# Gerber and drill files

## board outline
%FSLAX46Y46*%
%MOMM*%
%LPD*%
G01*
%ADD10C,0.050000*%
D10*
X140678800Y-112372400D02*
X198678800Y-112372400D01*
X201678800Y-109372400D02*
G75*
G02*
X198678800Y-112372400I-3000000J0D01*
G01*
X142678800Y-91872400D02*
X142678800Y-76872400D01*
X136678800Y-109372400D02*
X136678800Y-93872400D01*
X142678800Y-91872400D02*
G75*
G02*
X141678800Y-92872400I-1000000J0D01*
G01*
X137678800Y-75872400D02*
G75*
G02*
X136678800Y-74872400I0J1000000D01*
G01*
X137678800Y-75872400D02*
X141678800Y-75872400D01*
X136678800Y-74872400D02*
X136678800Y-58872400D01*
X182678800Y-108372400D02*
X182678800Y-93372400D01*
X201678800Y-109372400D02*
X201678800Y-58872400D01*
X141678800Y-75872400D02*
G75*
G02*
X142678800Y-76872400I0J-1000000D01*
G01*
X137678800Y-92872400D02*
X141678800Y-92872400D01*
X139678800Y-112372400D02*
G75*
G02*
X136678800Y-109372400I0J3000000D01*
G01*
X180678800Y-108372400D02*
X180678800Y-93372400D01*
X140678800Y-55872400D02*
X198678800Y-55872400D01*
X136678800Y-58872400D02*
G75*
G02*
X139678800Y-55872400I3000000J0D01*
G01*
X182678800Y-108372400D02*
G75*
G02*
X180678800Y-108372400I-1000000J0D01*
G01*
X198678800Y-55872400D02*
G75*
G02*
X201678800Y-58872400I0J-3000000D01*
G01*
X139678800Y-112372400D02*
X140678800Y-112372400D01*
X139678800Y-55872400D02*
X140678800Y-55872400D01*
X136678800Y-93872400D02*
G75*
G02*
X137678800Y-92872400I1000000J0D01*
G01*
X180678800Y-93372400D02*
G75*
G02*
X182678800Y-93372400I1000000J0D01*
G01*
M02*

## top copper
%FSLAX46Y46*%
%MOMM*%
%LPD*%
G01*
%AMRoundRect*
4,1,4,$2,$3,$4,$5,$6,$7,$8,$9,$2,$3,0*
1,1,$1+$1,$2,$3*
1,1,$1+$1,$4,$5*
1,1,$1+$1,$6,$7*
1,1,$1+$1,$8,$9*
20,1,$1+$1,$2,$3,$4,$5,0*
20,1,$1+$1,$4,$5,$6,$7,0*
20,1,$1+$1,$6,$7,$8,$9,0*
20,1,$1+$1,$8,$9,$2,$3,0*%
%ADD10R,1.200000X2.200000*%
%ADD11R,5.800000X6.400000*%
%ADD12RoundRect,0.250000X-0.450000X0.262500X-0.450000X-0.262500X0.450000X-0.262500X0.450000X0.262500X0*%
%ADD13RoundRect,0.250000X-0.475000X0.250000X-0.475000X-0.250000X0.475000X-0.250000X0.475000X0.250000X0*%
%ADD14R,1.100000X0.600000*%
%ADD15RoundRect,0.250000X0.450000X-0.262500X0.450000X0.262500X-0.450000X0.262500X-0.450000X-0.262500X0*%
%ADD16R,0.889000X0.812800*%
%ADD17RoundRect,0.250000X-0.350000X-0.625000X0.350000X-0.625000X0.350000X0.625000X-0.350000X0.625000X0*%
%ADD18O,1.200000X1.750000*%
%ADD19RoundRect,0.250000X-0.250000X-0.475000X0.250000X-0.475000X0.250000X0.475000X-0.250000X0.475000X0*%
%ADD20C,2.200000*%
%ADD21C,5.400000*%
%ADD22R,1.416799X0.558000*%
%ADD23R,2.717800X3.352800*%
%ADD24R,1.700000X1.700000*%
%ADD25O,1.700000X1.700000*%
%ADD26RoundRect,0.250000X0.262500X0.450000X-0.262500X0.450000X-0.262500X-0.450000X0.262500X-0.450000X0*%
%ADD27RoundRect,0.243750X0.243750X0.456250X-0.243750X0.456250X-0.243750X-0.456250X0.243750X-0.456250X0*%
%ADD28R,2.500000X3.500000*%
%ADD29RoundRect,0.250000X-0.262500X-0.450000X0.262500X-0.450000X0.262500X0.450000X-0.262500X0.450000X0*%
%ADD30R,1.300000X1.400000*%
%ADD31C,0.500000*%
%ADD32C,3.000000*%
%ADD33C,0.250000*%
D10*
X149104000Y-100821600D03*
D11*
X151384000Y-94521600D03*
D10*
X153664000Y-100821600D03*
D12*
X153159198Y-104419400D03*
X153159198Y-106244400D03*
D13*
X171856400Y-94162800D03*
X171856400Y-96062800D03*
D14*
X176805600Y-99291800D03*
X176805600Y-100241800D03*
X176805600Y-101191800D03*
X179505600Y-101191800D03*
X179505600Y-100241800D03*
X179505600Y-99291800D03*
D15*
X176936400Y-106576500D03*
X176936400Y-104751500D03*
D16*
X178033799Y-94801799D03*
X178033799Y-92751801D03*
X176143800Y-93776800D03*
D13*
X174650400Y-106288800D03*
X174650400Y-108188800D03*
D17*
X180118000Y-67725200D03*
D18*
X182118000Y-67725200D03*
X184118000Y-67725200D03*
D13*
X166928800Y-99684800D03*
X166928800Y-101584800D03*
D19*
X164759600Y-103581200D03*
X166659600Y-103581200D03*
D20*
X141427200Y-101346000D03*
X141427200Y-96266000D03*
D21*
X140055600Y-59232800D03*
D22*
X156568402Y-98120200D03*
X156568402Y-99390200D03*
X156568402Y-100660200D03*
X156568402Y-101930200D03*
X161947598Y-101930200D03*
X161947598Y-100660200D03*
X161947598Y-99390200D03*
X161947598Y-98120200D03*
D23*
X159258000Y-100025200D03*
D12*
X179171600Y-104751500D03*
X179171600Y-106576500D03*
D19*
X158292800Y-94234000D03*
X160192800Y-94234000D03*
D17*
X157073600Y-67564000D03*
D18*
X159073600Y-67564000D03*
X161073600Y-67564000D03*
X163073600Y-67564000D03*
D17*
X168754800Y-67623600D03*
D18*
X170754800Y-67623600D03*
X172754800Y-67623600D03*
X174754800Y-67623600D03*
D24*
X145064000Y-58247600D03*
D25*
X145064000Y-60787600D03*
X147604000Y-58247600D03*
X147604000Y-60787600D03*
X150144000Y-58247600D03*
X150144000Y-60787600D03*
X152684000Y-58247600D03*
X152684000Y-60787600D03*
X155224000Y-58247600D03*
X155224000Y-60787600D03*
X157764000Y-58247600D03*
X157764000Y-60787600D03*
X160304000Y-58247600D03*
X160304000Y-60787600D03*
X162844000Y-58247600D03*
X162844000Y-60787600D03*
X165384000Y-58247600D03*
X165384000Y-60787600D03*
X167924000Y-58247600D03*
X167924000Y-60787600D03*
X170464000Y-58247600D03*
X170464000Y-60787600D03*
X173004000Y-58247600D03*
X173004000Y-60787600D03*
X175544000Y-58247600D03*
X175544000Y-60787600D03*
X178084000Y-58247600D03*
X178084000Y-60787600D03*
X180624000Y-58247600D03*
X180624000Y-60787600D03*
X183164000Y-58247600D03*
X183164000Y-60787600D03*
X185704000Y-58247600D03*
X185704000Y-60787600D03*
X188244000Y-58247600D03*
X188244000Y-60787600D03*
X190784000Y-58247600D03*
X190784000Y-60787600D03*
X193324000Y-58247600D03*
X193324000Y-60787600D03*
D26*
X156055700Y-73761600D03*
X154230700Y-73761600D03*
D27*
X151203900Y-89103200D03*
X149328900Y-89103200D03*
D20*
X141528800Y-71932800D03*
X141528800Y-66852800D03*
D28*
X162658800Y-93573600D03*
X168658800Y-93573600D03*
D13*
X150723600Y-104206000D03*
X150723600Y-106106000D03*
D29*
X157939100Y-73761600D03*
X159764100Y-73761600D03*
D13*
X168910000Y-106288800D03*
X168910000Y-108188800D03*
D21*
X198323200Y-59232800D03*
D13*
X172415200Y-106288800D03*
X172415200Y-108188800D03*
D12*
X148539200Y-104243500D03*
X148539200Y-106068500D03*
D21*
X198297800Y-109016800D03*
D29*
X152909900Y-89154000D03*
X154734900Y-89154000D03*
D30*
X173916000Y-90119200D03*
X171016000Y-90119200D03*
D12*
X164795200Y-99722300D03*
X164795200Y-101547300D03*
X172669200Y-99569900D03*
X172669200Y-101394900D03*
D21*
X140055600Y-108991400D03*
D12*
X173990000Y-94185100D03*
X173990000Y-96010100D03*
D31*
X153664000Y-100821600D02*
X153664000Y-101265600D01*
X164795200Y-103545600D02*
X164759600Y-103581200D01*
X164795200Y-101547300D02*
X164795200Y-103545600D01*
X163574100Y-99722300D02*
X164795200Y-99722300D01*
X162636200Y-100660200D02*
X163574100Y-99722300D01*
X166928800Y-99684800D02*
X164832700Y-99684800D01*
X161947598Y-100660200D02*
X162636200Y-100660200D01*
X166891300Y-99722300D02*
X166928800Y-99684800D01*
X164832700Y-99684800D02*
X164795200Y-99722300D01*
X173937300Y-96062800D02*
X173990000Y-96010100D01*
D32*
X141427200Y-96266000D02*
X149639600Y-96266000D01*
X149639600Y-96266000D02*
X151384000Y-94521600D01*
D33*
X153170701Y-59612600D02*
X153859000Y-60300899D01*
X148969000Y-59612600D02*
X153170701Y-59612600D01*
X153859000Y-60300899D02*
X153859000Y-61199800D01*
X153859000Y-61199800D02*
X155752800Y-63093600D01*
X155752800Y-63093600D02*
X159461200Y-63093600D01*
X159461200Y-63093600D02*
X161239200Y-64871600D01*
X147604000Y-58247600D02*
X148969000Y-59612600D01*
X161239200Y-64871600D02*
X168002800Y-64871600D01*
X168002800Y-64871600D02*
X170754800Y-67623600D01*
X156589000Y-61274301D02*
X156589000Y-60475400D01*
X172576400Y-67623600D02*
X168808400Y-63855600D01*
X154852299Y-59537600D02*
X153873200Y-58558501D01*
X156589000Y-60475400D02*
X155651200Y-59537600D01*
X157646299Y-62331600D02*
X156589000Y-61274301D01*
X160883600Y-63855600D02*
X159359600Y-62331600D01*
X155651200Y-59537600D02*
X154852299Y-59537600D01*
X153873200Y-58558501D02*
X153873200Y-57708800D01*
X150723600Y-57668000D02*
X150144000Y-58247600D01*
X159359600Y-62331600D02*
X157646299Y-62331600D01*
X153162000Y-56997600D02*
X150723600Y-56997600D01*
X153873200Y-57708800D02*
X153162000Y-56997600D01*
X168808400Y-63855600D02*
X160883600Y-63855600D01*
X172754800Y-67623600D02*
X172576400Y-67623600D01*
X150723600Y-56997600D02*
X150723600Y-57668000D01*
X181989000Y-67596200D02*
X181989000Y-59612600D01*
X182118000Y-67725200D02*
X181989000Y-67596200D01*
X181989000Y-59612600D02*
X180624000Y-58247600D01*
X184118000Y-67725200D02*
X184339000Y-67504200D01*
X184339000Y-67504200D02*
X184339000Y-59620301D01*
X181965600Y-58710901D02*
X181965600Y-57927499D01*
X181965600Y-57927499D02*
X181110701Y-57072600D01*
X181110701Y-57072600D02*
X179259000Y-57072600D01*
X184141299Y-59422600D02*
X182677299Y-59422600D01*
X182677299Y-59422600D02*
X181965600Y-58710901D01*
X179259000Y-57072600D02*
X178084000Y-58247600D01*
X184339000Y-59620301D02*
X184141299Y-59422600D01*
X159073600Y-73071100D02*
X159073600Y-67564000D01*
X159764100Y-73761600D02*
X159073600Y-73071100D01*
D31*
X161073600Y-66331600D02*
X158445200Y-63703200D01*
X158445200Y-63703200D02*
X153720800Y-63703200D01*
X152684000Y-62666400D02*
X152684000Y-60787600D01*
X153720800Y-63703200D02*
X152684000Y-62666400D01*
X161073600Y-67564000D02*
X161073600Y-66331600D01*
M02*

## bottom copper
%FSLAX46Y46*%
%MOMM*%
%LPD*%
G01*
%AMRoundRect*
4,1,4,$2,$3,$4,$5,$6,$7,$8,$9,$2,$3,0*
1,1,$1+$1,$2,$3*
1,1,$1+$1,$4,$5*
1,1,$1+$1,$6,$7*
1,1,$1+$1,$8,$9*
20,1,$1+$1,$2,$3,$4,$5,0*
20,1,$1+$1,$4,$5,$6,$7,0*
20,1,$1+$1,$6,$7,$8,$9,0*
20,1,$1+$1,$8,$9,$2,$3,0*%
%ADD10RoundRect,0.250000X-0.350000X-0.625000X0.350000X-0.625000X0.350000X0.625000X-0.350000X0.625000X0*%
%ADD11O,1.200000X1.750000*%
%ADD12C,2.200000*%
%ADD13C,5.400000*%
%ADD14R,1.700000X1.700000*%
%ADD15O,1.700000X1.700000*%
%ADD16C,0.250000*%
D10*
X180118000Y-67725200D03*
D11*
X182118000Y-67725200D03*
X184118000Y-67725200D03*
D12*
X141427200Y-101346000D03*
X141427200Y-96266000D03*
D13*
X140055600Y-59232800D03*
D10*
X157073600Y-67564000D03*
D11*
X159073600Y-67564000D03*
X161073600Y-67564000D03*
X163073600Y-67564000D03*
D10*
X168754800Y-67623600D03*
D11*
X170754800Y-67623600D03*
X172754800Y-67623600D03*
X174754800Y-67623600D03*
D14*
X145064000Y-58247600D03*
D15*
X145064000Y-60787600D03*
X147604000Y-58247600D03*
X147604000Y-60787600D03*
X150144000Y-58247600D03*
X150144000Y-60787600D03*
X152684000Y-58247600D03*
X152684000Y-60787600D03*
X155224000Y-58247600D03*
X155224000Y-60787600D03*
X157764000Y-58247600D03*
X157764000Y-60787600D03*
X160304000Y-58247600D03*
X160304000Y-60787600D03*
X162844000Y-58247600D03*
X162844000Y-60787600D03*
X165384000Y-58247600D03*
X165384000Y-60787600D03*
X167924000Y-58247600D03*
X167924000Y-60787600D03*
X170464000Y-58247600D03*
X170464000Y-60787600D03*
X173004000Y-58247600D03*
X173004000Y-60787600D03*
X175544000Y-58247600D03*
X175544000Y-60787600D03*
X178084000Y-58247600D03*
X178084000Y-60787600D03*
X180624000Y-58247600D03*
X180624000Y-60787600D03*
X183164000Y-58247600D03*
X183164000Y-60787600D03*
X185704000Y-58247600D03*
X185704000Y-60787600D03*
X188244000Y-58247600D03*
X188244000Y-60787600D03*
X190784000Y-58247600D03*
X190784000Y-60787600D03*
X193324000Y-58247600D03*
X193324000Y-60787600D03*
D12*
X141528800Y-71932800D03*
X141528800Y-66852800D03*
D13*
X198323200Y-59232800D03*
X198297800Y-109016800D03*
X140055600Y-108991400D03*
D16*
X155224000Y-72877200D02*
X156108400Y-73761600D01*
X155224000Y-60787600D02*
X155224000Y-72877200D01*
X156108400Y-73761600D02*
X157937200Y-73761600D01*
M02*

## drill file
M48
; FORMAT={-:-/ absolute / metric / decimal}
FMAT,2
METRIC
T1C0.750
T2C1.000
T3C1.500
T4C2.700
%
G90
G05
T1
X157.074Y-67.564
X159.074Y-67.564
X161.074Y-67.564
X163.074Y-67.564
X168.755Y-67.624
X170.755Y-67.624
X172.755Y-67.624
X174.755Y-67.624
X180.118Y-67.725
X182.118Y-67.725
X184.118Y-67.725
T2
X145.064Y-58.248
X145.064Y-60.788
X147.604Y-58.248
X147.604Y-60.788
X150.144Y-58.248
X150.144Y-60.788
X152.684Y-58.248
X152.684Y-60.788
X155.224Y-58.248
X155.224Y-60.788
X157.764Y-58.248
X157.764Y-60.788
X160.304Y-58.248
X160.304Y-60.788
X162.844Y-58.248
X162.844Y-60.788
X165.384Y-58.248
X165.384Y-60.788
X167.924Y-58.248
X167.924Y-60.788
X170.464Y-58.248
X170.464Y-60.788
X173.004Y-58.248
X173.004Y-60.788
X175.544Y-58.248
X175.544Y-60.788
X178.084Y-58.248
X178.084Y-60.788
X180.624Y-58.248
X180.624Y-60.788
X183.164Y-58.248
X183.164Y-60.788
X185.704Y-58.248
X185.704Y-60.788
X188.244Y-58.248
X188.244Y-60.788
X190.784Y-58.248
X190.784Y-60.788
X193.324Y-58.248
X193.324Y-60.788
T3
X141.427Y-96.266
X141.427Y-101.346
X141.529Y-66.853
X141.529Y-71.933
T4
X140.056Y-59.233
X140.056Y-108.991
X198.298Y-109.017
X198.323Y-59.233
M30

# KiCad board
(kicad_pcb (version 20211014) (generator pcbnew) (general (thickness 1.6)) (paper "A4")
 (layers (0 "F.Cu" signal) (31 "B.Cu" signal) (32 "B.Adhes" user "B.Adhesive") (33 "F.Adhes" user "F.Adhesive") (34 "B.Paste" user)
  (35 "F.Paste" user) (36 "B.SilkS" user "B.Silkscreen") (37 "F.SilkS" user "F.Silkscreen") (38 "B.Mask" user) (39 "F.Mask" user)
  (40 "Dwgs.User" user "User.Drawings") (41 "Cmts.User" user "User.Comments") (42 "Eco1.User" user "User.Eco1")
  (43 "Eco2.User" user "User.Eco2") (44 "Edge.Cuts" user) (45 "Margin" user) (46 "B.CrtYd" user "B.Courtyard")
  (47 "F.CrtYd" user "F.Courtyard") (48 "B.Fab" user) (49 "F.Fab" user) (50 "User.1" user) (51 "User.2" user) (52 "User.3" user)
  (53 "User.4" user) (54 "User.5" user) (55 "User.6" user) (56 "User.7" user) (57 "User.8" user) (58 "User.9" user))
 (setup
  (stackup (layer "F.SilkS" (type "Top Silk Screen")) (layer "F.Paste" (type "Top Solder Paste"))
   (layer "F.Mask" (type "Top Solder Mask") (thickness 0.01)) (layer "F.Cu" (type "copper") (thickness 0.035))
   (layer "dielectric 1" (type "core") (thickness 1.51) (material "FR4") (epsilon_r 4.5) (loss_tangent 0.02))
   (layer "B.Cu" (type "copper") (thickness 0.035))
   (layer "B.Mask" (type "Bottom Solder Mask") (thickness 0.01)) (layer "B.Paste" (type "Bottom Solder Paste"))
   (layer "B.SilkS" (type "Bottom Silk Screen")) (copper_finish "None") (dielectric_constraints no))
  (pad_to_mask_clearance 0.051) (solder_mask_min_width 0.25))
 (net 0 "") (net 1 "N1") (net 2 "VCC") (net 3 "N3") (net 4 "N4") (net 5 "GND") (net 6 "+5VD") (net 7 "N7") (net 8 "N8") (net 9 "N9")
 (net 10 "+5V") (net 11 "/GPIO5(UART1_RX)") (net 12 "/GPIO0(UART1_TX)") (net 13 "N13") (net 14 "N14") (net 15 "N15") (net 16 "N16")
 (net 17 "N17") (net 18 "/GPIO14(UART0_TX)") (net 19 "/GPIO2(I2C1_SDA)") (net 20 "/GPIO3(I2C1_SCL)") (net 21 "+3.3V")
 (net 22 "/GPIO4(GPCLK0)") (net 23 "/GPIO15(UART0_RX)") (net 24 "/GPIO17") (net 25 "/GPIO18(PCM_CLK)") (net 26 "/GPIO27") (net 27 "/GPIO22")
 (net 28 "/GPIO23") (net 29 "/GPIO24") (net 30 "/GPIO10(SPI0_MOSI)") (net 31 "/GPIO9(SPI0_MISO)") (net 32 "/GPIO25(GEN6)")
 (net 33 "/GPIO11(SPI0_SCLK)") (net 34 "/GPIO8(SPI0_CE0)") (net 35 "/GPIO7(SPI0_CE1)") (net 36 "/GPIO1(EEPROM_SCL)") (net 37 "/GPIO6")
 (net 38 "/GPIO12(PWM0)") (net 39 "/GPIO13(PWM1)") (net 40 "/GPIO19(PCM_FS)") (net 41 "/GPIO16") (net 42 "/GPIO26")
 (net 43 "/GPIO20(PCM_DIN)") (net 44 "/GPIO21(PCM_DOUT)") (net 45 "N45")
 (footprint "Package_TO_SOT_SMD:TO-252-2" (layer "F.Cu") (at 151.384 96.6216 90)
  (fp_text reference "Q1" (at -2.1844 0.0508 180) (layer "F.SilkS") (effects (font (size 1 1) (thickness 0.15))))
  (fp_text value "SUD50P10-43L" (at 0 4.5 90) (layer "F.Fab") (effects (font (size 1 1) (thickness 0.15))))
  (pad "" smd rect (at 0.425 1.525 90) (size 3.05 2.75) (layers "F.Paste"))
  (pad "" smd rect (at 3.775 1.525 90) (size 3.05 2.75) (layers "F.Paste"))
  (pad "" smd rect (at 3.775 -1.525 90) (size 3.05 2.75) (layers "F.Paste"))
  (pad "" smd rect (at 0.425 -1.525 90) (size 3.05 2.75) (layers "F.Paste"))
  (pad "1" smd rect (at -4.2 -2.28 90) (size 2.2 1.2) (layers "F.Cu" "F.Paste" "F.Mask") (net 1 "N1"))
  (pad "2" smd rect (at 2.1 0 90) (size 6.4 5.8) (layers "F.Cu" "F.Mask") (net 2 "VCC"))
  (pad "3" smd rect (at -4.2 2.28 90) (size 2.2 1.2) (layers "F.Cu" "F.Paste" "F.Mask") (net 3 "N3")))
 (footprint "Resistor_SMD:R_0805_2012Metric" (layer "F.Cu") (at 153.159198 105.3319 -90)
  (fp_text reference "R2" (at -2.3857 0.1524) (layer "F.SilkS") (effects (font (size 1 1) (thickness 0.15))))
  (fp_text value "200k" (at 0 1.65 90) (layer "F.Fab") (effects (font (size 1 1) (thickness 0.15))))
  (pad "1" smd roundrect (at -0.9125 0 270) (size 1.025 1.4) (layers "F.Cu" "F.Paste" "F.Mask") (roundrect_rratio 0.243902) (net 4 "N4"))
  (pad "2" smd roundrect (at 0.9125 0 270) (size 1.025 1.4) (layers "F.Cu" "F.Paste" "F.Mask") (roundrect_rratio 0.243902) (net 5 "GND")))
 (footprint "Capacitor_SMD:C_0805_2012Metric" (layer "F.Cu") (at 171.8564 95.1128 -90)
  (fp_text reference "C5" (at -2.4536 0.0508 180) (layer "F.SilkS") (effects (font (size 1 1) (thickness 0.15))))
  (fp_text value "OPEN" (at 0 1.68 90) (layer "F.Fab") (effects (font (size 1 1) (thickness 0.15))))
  (pad "1" smd roundrect (at -0.95 0 270) (size 1 1.45) (layers "F.Cu" "F.Paste" "F.Mask") (roundrect_rratio 0.25) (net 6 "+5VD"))
  (pad "2" smd roundrect (at 0.95 0 270) (size 1 1.45) (layers "F.Cu" "F.Paste" "F.Mask") (roundrect_rratio 0.25) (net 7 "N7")))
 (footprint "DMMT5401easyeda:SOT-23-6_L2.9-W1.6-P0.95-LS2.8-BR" (layer "F.Cu") (at 178.1556 100.2418 180)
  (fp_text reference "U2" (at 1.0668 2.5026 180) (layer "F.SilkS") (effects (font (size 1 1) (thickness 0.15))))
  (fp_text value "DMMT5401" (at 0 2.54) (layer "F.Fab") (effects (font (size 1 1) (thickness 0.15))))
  (pad "1" smd rect (at 1.35 0.95 180) (size 1.1 0.6) (layers "F.Cu" "F.Paste" "F.Mask") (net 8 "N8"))
  (pad "2" smd rect (at 1.35 0 180) (size 1.1 0.6) (layers "F.Cu" "F.Paste" "F.Mask") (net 8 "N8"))
  (pad "3" smd rect (at 1.35 -0.95 180) (size 1.1 0.6) (layers "F.Cu" "F.Paste" "F.Mask") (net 8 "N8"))
  (pad "4" smd rect (at -1.35 -0.95 180) (size 1.1 0.6) (layers "F.Cu" "F.Paste" "F.Mask") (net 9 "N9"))
  (pad "5" smd rect (at -1.35 0 180) (size 1.1 0.6) (layers "F.Cu" "F.Paste" "F.Mask") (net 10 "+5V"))
  (pad "6" smd rect (at -1.35 0.95 180) (size 1.1 0.6) (layers "F.Cu" "F.Paste" "F.Mask") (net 6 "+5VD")))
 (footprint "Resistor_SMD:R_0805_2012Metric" (layer "F.Cu") (at 176.9364 105.664 90)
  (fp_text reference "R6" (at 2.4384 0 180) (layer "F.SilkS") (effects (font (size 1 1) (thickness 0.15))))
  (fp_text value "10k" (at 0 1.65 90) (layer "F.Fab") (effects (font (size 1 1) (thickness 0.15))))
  (pad "1" smd roundrect (at -0.9125 0 90) (size 1.025 1.4) (layers "F.Cu" "F.Paste" "F.Mask") (roundrect_rratio 0.243902) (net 5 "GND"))
  (pad "2" smd roundrect (at 0.9125 0 90) (size 1.025 1.4) (layers "F.Cu" "F.Paste" "F.Mask") (roundrect_rratio 0.243902) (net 8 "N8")))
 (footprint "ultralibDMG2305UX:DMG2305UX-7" (layer "F.Cu") (at 177.0888 93.7768 90)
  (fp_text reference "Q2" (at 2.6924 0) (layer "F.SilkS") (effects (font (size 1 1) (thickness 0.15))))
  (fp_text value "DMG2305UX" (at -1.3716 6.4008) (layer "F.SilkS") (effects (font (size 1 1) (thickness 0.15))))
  (pad "1" smd rect (at -1.024999 0.944999 90) (size 0.8128 0.889) (layers "F.Cu" "F.Paste" "F.Mask") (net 9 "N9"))
  (pad "2" smd rect (at 1.024999 0.944999 90) (size 0.8128 0.889) (layers "F.Cu" "F.Paste" "F.Mask") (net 10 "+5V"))
  (pad "3" smd rect (at 0 -0.945 90) (size 0.8128 0.889) (layers "F.Cu" "F.Paste" "F.Mask") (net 6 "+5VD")))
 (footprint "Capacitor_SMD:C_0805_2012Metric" (layer "F.Cu") (at 174.6504 107.2388 -90)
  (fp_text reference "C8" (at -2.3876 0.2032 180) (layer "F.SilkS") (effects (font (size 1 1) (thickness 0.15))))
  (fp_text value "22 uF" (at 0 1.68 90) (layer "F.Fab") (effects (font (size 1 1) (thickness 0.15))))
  (pad "1" smd roundrect (at -0.95 0 270) (size 1 1.45) (layers "F.Cu" "F.Paste" "F.Mask") (roundrect_rratio 0.25) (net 6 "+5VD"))
  (pad "2" smd roundrect (at 0.95 0 270) (size 1 1.45) (layers "F.Cu" "F.Paste" "F.Mask") (roundrect_rratio 0.25) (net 5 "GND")))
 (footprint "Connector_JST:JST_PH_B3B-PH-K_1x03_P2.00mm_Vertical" (layer "F.Cu") (at 180.118 67.7252)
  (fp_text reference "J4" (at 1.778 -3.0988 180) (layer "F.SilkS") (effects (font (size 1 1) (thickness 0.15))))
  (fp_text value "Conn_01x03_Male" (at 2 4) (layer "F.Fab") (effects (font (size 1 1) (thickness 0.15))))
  (pad "1" thru_hole roundrect (at 0 0) (size 1.2 1.75) (drill 0.75) (layers *.Cu *.Mask) (roundrect_rratio 0.208333) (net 5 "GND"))
  (pad "2" thru_hole oval (at 2 0) (size 1.2 1.75) (drill 0.75) (layers *.Cu *.Mask) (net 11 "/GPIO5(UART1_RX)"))
  (pad "3" thru_hole oval (at 4 0) (size 1.2 1.75) (drill 0.75) (layers *.Cu *.Mask) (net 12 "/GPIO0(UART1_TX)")))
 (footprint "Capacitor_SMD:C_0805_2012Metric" (layer "F.Cu") (at 166.9288 100.6348 -90)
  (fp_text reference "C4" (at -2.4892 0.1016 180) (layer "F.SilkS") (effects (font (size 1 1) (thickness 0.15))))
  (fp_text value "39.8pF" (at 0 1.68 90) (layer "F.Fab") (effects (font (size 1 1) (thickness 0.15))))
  (pad "1" smd roundrect (at -0.95 0 270) (size 1 1.45) (layers "F.Cu" "F.Paste" "F.Mask") (roundrect_rratio 0.25) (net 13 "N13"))
  (pad "2" smd roundrect (at 0.95 0 270) (size 1 1.45) (layers "F.Cu" "F.Paste" "F.Mask") (roundrect_rratio 0.25) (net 5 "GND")))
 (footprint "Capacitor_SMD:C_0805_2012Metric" (layer "F.Cu") (at 165.7096 103.5812)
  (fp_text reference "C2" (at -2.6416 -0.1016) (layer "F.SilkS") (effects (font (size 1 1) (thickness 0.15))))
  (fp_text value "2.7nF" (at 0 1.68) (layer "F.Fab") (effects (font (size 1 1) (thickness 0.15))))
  (pad "1" smd roundrect (at -0.95 0) (size 1 1.45) (layers "F.Cu" "F.Paste" "F.Mask") (roundrect_rratio 0.25) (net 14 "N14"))
  (pad "2" smd roundrect (at 0.95 0) (size 1 1.45) (layers "F.Cu" "F.Paste" "F.Mask") (roundrect_rratio 0.25) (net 5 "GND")))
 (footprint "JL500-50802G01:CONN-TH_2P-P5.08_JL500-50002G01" (layer "F.Cu") (at 141.4272 98.806 90)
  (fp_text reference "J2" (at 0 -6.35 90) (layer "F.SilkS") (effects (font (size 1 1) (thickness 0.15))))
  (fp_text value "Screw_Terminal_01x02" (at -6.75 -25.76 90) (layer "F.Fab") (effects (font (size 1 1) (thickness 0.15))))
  (pad "1" thru_hole circle (at -2.54 0 90) (size 2.2 2.2) (drill 1.500022) (layers *.Cu *.Mask) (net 5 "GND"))
  (pad "2" thru_hole circle (at 2.54 0 90) (size 2.2 2.2) (drill 1.500022) (layers *.Cu *.Mask) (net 2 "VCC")))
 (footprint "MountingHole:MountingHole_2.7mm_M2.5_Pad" (layer "F.Cu") (at 140.0556 59.2328)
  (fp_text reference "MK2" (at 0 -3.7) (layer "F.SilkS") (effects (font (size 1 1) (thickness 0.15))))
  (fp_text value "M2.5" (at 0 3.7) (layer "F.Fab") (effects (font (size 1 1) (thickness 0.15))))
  (pad "1" thru_hole circle (at 0 0) (size 5.4 5.4) (drill 2.7) (layers *.Cu *.Mask)))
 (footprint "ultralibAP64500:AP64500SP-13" (layer "F.Cu") (at 159.258 100.0252)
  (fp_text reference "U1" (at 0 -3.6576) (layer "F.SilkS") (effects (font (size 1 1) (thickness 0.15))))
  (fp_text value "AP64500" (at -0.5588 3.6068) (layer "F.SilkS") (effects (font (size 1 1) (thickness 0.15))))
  (pad "1" smd rect (at -2.689598 -1.905) (size 1.416799 0.558) (layers "F.Cu" "F.Paste" "F.Mask") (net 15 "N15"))
  (pad "2" smd rect (at -2.689598 -0.635) (size 1.416799 0.558) (layers "F.Cu" "F.Paste" "F.Mask") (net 3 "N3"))
  (pad "3" smd rect (at -2.689598 0.635) (size 1.416799 0.558) (layers "F.Cu" "F.Paste" "F.Mask") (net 3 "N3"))
  (pad "4" smd rect (at -2.689598 1.905) (size 1.416799 0.558) (layers "F.Cu" "F.Paste" "F.Mask") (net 4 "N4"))
  (pad "5" smd rect (at 2.689598 1.905) (size 1.416799 0.558) (layers "F.Cu" "F.Paste" "F.Mask") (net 7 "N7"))
  (pad "6" smd rect (at 2.689598 0.635) (size 1.416799 0.558) (layers "F.Cu" "F.Paste" "F.Mask") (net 13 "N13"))
  (pad "7" smd rect (at 2.689598 -0.635) (size 1.416799 0.558) (layers "F.Cu" "F.Paste" "F.Mask") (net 5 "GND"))
  (pad "8" smd rect (at 2.689598 -1.905) (size 1.416799 0.558) (layers "F.Cu" "F.Paste" "F.Mask") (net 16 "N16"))
  (pad "EPAD" smd rect (at 0 0) (size 2.7178 3.3528) (layers "F.Cu" "F.Paste" "F.Mask")))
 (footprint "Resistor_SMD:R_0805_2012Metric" (layer "F.Cu") (at 179.1716 105.664 -90)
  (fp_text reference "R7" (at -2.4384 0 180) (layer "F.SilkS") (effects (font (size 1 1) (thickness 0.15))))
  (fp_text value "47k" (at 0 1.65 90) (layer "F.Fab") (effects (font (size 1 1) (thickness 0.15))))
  (pad "1" smd roundrect (at -0.9125 0 270) (size 1.025 1.4) (layers "F.Cu" "F.Paste" "F.Mask") (roundrect_rratio 0.243902) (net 9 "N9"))
  (pad "2" smd roundrect (at 0.9125 0 270) (size 1.025 1.4) (layers "F.Cu" "F.Paste" "F.Mask") (roundrect_rratio 0.243902) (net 5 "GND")))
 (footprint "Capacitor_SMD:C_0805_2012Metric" (layer "F.Cu") (at 159.2428 94.234)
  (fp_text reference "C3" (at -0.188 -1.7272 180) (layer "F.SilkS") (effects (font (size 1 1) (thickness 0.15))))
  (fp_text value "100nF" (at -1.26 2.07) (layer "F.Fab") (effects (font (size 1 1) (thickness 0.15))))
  (pad "1" smd roundrect (at -0.95 0) (size 1 1.45) (layers "F.Cu" "F.Paste" "F.Mask") (roundrect_rratio 0.25) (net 15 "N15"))
  (pad "2" smd roundrect (at 0.95 0) (size 1 1.45) (layers "F.Cu" "F.Paste" "F.Mask") (roundrect_rratio 0.25) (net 16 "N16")))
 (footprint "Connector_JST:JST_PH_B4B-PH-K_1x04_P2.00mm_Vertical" (layer "F.Cu") (at 157.0736 67.564)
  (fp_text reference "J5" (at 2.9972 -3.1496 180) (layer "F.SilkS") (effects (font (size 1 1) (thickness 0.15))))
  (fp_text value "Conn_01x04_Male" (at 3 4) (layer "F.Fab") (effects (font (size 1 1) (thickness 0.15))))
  (pad "1" thru_hole roundrect (at 0 0) (size 1.2 1.75) (drill 0.75) (layers *.Cu *.Mask) (roundrect_rratio 0.208333) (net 5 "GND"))
  (pad "2" thru_hole oval (at 2 0) (size 1.2 1.75) (drill 0.75) (layers *.Cu *.Mask) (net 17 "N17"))
  (pad "3" thru_hole oval (at 4 0) (size 1.2 1.75) (drill 0.75) (layers *.Cu *.Mask) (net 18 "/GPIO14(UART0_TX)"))
  (pad "4" thru_hole oval (at 6 0) (size 1.2 1.75) (drill 0.75) (layers *.Cu *.Mask) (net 10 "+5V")))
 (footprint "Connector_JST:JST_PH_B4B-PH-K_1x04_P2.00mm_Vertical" (layer "F.Cu") (at 168.7548 67.6236)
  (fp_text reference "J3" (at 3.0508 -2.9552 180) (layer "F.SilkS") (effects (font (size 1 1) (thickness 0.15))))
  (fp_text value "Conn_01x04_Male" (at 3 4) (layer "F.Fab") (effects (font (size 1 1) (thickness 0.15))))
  (pad "1" thru_hole roundrect (at 0 0) (size 1.2 1.75) (drill 0.75) (layers *.Cu *.Mask) (roundrect_rratio 0.208333) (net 5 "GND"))
  (pad "2" thru_hole oval (at 2 0) (size 1.2 1.75) (drill 0.75) (layers *.Cu *.Mask) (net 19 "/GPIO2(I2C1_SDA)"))
  (pad "3" thru_hole oval (at 4 0) (size 1.2 1.75) (drill 0.75) (layers *.Cu *.Mask) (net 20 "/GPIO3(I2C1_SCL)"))
  (pad "4" thru_hole oval (at 6 0) (size 1.2 1.75) (drill 0.75) (layers *.Cu *.Mask) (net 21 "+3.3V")))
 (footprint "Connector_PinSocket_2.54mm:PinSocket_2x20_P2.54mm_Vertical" (layer "F.Cu") (at 145.064 58.2476 90)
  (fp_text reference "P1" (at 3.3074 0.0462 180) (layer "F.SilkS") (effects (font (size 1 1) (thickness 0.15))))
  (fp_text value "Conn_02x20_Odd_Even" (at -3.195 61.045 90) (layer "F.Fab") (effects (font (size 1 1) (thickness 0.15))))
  (pad "1" thru_hole rect (at 0 0 90) (size 1.7 1.7) (drill 1) (layers *.Cu *.Mask) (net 21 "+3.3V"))
  (pad "2" thru_hole oval (at -2.54 0 90) (size 1.7 1.7) (drill 1) (layers *.Cu *.Mask) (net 10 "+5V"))
  (pad "3" thru_hole oval (at 0 2.54 90) (size 1.7 1.7) (drill 1) (layers *.Cu *.Mask) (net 19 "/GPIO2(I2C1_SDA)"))
  (pad "4" thru_hole oval (at -2.54 2.54 90) (size 1.7 1.7) (drill 1) (layers *.Cu *.Mask) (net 10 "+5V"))
  (pad "5" thru_hole oval (at 0 5.08 90) (size 1.7 1.7) (drill 1) (layers *.Cu *.Mask) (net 20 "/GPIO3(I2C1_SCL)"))
  (pad "6" thru_hole oval (at -2.54 5.08 90) (size 1.7 1.7) (drill 1) (layers *.Cu *.Mask) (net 5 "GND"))
  (pad "7" thru_hole oval (at 0 7.62 90) (size 1.7 1.7) (drill 1) (layers *.Cu *.Mask) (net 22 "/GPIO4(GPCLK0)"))
  (pad "8" thru_hole oval (at -2.54 7.62 90) (size 1.7 1.7) (drill 1) (layers *.Cu *.Mask) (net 18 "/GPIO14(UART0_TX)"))
  (pad "9" thru_hole oval (at 0 10.16 90) (size 1.7 1.7) (drill 1) (layers *.Cu *.Mask) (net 5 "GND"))
  (pad "10" thru_hole oval (at -2.54 10.16 90) (size 1.7 1.7) (drill 1) (layers *.Cu *.Mask) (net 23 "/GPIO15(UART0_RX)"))
  (pad "11" thru_hole oval (at 0 12.7 90) (size 1.7 1.7) (drill 1) (layers *.Cu *.Mask) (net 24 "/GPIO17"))
  (pad "12" thru_hole oval (at -2.54 12.7 90) (size 1.7 1.7) (drill 1) (layers *.Cu *.Mask) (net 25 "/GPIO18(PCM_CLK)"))
  (pad "13" thru_hole oval (at 0 15.24 90) (size 1.7 1.7) (drill 1) (layers *.Cu *.Mask) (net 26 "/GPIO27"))
  (pad "14" thru_hole oval (at -2.54 15.24 90) (size 1.7 1.7) (drill 1) (layers *.Cu *.Mask) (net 5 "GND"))
  (pad "15" thru_hole oval (at 0 17.78 90) (size 1.7 1.7) (drill 1) (layers *.Cu *.Mask) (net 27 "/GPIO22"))
  (pad "16" thru_hole oval (at -2.54 17.78 90) (size 1.7 1.7) (drill 1) (layers *.Cu *.Mask) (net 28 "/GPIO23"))
  (pad "17" thru_hole oval (at 0 20.32 90) (size 1.7 1.7) (drill 1) (layers *.Cu *.Mask) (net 21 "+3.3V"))
  (pad "18" thru_hole oval (at -2.54 20.32 90) (size 1.7 1.7) (drill 1) (layers *.Cu *.Mask) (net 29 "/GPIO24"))
  (pad "19" thru_hole oval (at 0 22.86 90) (size 1.7 1.7) (drill 1) (layers *.Cu *.Mask) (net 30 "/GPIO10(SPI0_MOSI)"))
  (pad "20" thru_hole oval (at -2.54 22.86 90) (size 1.7 1.7) (drill 1) (layers *.Cu *.Mask) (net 5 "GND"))
  (pad "21" thru_hole oval (at 0 25.4 90) (size 1.7 1.7) (drill 1) (layers *.Cu *.Mask) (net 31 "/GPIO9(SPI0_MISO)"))
  (pad "22" thru_hole oval (at -2.54 25.4 90) (size 1.7 1.7) (drill 1) (layers *.Cu *.Mask) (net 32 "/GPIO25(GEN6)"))
  (pad "23" thru_hole oval (at 0 27.94 90) (size 1.7 1.7) (drill 1) (layers *.Cu *.Mask) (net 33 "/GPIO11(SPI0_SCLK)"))
  (pad "24" thru_hole oval (at -2.54 27.94 90) (size 1.7 1.7) (drill 1) (layers *.Cu *.Mask) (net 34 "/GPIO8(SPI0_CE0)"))
  (pad "25" thru_hole oval (at 0 30.48 90) (size 1.7 1.7) (drill 1) (layers *.Cu *.Mask) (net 5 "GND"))
  (pad "26" thru_hole oval (at -2.54 30.48 90) (size 1.7 1.7) (drill 1) (layers *.Cu *.Mask) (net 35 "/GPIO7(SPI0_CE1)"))
  (pad "27" thru_hole oval (at 0 33.02 90) (size 1.7 1.7) (drill 1) (layers *.Cu *.Mask) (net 12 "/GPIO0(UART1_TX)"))
  (pad "28" thru_hole oval (at -2.54 33.02 90) (size 1.7 1.7) (drill 1) (layers *.Cu *.Mask) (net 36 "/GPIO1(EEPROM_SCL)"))
  (pad "29" thru_hole oval (at 0 35.56 90) (size 1.7 1.7) (drill 1) (layers *.Cu *.Mask) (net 11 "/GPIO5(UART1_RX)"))
  (pad "30" thru_hole oval (at -2.54 35.56 90) (size 1.7 1.7) (drill 1) (layers *.Cu *.Mask) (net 5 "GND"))
  (pad "31" thru_hole oval (at 0 38.1 90) (size 1.7 1.7) (drill 1) (layers *.Cu *.Mask) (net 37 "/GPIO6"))
  (pad "32" thru_hole oval (at -2.54 38.1 90) (size 1.7 1.7) (drill 1) (layers *.Cu *.Mask) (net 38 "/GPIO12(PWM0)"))
  (pad "33" thru_hole oval (at 0 40.64 90) (size 1.7 1.7) (drill 1) (layers *.Cu *.Mask) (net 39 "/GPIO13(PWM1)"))
  (pad "34" thru_hole oval (at -2.54 40.64 90) (size 1.7 1.7) (drill 1) (layers *.Cu *.Mask) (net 5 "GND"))
  (pad "35" thru_hole oval (at 0 43.18 90) (size 1.7 1.7) (drill 1) (layers *.Cu *.Mask) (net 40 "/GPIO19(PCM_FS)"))
  (pad "36" thru_hole oval (at -2.54 43.18 90) (size 1.7 1.7) (drill 1) (layers *.Cu *.Mask) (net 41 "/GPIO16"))
  (pad "37" thru_hole oval (at 0 45.72 90) (size 1.7 1.7) (drill 1) (layers *.Cu *.Mask) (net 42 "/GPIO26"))
  (pad "38" thru_hole oval (at -2.54 45.72 90) (size 1.7 1.7) (drill 1) (layers *.Cu *.Mask) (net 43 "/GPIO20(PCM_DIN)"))
  (pad "39" thru_hole oval (at 0 48.26 90) (size 1.7 1.7) (drill 1) (layers *.Cu *.Mask) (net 5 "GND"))
  (pad "40" thru_hole oval (at -2.54 48.26 90) (size 1.7 1.7) (drill 1) (layers *.Cu *.Mask) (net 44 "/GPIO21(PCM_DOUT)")))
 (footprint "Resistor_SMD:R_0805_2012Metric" (layer "F.Cu") (at 155.1432 73.7616 180)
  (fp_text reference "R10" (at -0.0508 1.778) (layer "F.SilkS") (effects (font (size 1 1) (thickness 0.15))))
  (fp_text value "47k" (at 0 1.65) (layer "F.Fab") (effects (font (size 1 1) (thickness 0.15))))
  (pad "1" smd roundrect (at -0.9125 0 180) (size 1.025 1.4) (layers "F.Cu" "F.Paste" "F.Mask") (roundrect_rratio 0.243902)
   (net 23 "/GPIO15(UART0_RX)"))
  (pad "2" smd roundrect (at 0.9125 0 180) (size 1.025 1.4) (layers "F.Cu" "F.Paste" "F.Mask") (roundrect_rratio 0.243902) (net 5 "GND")))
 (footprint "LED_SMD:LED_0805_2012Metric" (layer "F.Cu") (at 150.2664 89.1032 180)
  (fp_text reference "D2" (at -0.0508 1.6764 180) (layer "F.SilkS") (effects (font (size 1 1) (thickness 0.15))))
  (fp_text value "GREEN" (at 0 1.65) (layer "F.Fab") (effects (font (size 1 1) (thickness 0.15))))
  (pad "1" smd roundrect (at -0.9375 0 180) (size 0.975 1.4) (layers "F.Cu" "F.Paste" "F.Mask") (roundrect_rratio 0.25) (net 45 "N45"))
  (pad "2" smd roundrect (at 0.9375 0 180) (size 0.975 1.4) (layers "F.Cu" "F.Paste" "F.Mask") (roundrect_rratio 0.25) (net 6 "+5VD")))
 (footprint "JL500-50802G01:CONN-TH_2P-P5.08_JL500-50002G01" (layer "F.Cu") (at 141.5288 69.3928 90)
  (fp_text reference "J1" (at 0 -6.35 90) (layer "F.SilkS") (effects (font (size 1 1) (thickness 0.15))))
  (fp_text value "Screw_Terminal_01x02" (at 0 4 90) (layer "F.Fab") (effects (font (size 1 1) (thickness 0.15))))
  (pad "1" thru_hole circle (at -2.54 0 90) (size 2.2 2.2) (drill 1.500022) (layers *.Cu *.Mask) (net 5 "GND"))
  (pad "2" thru_hole circle (at 2.54 0 90) (size 2.2 2.2) (drill 1.500022) (layers *.Cu *.Mask) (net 10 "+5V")))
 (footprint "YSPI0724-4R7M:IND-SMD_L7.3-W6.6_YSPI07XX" (layer "F.Cu") (at 165.6588 93.5736)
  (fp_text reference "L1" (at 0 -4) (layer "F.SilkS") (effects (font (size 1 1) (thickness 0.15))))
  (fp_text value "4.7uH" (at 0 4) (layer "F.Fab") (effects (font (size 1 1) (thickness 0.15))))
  (pad "1" smd rect (at -3 0) (size 2.5 3.5) (layers "F.Cu" "F.Paste" "F.Mask") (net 16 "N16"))
  (pad "2" smd rect (at 3 0) (size 2.5 3.5) (layers "F.Cu" "F.Paste" "F.Mask") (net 6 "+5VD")))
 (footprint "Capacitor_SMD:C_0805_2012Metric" (layer "F.Cu") (at 150.7236 105.156 -90)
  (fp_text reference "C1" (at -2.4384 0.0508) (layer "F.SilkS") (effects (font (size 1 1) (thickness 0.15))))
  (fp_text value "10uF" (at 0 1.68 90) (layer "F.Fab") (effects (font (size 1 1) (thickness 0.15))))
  (pad "1" smd roundrect (at -0.95 0 270) (size 1 1.45) (layers "F.Cu" "F.Paste" "F.Mask") (roundrect_rratio 0.25) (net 3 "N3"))
  (pad "2" smd roundrect (at 0.95 0 270) (size 1 1.45) (layers "F.Cu" "F.Paste" "F.Mask") (roundrect_rratio 0.25) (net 5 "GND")))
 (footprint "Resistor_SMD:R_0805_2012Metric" (layer "F.Cu") (at 158.8516 73.7616)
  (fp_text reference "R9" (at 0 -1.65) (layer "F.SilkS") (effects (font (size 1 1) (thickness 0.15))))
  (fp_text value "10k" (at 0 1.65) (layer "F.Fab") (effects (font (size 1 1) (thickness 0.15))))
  (pad "1" smd roundrect (at -0.9125 0) (size 1.025 1.4) (layers "F.Cu" "F.Paste" "F.Mask") (roundrect_rratio 0.243902)
   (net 23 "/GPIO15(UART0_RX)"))
  (pad "2" smd roundrect (at 0.9125 0) (size 1.025 1.4) (layers "F.Cu" "F.Paste" "F.Mask") (roundrect_rratio 0.243902) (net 17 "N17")))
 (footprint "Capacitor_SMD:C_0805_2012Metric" (layer "F.Cu") (at 168.91 107.2388 -90)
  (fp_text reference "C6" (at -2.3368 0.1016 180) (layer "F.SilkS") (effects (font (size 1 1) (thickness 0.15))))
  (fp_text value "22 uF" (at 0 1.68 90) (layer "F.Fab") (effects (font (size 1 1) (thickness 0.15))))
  (pad "1" smd roundrect (at -0.95 0 270) (size 1 1.45) (layers "F.Cu" "F.Paste" "F.Mask") (roundrect_rratio 0.25) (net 6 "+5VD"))
  (pad "2" smd roundrect (at 0.95 0 270) (size 1 1.45) (layers "F.Cu" "F.Paste" "F.Mask") (roundrect_rratio 0.25) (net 5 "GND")))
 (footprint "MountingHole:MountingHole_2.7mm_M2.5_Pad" (layer "F.Cu") (at 198.3232 59.2328)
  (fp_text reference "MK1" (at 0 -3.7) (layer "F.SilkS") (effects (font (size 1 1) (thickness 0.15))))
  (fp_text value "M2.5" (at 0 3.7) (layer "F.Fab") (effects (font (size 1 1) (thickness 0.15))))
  (pad "1" thru_hole circle (at 0 0) (size 5.4 5.4) (drill 2.7) (layers *.Cu *.Mask)))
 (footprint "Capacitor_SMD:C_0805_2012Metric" (layer "F.Cu") (at 172.4152 107.2388 -90)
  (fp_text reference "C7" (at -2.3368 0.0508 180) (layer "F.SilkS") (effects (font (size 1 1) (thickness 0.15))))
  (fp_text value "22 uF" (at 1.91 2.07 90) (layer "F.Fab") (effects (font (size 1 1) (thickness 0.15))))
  (pad "1" smd roundrect (at -0.95 0 270) (size 1 1.45) (layers "F.Cu" "F.Paste" "F.Mask") (roundrect_rratio 0.25) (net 6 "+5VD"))
  (pad "2" smd roundrect (at 0.95 0 270) (size 1 1.45) (layers "F.Cu" "F.Paste" "F.Mask") (roundrect_rratio 0.25) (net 5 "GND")))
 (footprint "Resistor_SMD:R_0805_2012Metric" (layer "F.Cu") (at 148.5392 105.156 -90)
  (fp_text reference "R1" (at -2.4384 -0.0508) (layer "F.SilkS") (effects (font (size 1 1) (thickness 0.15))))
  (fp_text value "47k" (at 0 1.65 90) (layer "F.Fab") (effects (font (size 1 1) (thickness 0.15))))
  (pad "1" smd roundrect (at -0.9125 0 270) (size 1.025 1.4) (layers "F.Cu" "F.Paste" "F.Mask") (roundrect_rratio 0.243902) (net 1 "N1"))
  (pad "2" smd roundrect (at 0.9125 0 270) (size 1.025 1.4) (layers "F.Cu" "F.Paste" "F.Mask") (roundrect_rratio 0.243902) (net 5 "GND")))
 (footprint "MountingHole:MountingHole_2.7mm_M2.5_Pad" (layer "F.Cu") (at 198.2978 109.0168)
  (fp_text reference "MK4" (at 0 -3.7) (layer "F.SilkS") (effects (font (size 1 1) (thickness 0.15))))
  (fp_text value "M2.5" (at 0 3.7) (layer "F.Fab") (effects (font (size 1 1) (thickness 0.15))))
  (pad "1" thru_hole circle (at 0 0) (size 5.4 5.4) (drill 2.7) (layers *.Cu *.Mask)))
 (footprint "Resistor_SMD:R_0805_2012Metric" (layer "F.Cu") (at 153.8224 89.154)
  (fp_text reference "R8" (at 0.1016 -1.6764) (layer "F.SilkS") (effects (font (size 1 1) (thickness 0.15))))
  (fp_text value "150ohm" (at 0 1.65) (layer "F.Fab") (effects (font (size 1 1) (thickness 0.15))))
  (pad "1" smd roundrect (at -0.9125 0) (size 1.025 1.4) (layers "F.Cu" "F.Paste" "F.Mask") (roundrect_rratio 0.243902) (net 45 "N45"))
  (pad "2" smd roundrect (at 0.9125 0) (size 1.025 1.4) (layers "F.Cu" "F.Paste" "F.Mask") (roundrect_rratio 0.243902) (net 5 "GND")))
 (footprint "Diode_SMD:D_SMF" (layer "F.Cu") (at 172.466 90.1192 180)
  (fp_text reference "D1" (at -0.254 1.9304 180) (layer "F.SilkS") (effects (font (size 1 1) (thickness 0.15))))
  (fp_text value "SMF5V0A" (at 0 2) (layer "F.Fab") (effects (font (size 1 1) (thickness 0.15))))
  (pad "1" smd rect (at -1.45 0 180) (size 1.3 1.4) (layers "F.Cu" "F.Paste" "F.Mask") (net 5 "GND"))
  (pad "2" smd rect (at 1.45 0 180) (size 1.3 1.4) (layers "F.Cu" "F.Paste" "F.Mask") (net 6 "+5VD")))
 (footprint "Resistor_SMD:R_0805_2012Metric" (layer "F.Cu") (at 164.7952 100.6348 -90)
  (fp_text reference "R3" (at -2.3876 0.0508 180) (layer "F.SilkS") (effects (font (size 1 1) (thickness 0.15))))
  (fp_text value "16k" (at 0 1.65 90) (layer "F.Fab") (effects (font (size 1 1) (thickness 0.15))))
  (pad "1" smd roundrect (at -0.9125 0 270) (size 1.025 1.4) (layers "F.Cu" "F.Paste" "F.Mask") (roundrect_rratio 0.243902) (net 13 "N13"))
  (pad "2" smd roundrect (at 0.9125 0 270) (size 1.025 1.4) (layers "F.Cu" "F.Paste" "F.Mask") (roundrect_rratio 0.243902) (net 14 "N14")))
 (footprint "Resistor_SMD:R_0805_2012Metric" (layer "F.Cu") (at 172.6692 100.4824 -90)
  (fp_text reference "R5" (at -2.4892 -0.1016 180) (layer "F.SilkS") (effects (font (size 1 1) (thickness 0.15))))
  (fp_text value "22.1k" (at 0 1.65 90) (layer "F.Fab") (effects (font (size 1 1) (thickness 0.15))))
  (pad "1" smd roundrect (at -0.9125 0 270) (size 1.025 1.4) (layers "F.Cu" "F.Paste" "F.Mask") (roundrect_rratio 0.243902) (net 7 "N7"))
  (pad "2" smd roundrect (at 0.9125 0 270) (size 1.025 1.4) (layers "F.Cu" "F.Paste" "F.Mask") (roundrect_rratio 0.243902) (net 5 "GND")))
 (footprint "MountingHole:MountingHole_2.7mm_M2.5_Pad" (layer "F.Cu") (at 140.0556 108.9914)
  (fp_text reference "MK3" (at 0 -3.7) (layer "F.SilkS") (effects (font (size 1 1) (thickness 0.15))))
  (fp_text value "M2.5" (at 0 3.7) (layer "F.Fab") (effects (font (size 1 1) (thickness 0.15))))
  (pad "1" thru_hole circle (at 0 0) (size 5.4 5.4) (drill 2.7) (layers *.Cu *.Mask)))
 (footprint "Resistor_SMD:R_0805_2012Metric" (layer "F.Cu") (at 173.99 95.0976 -90)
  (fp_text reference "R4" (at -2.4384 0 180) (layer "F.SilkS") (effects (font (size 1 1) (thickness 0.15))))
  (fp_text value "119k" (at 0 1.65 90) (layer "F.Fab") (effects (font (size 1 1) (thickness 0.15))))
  (pad "1" smd roundrect (at -0.9125 0 270) (size 1.025 1.4) (layers "F.Cu" "F.Paste" "F.Mask") (roundrect_rratio 0.243902) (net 6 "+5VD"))
  (pad "2" smd roundrect (at 0.9125 0 270) (size 1.025 1.4) (layers "F.Cu" "F.Paste" "F.Mask") (roundrect_rratio 0.243902) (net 7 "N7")))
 (gr_line (start 140.6788 112.3724) (end 198.6788 112.3724) (layer "Edge.Cuts") (width 0.05))
 (gr_arc (start 201.6788 109.3724) (mid 200.80012 111.49372) (end 198.6788 112.3724) (layer "Edge.Cuts") (width 0.05))
 (gr_line (start 142.6788 91.8724) (end 142.6788 76.8724) (layer "Edge.Cuts") (width 0.05))
 (gr_line (start 136.6788 109.3724) (end 136.6788 93.8724) (layer "Edge.Cuts") (width 0.05))
 (gr_arc (start 142.6788 91.8724) (mid 142.385907 92.579507) (end 141.6788 92.8724) (layer "Edge.Cuts") (width 0.05))
 (gr_arc (start 137.6788 75.8724) (mid 136.971693 75.579507) (end 136.6788 74.8724) (layer "Edge.Cuts") (width 0.05))
 (gr_line (start 137.6788 75.8724) (end 141.6788 75.8724) (layer "Edge.Cuts") (width 0.05))
 (gr_line (start 136.6788 74.8724) (end 136.6788 58.8724) (layer "Edge.Cuts") (width 0.05))
 (gr_line (start 182.6788 108.3724) (end 182.6788 93.3724) (layer "Edge.Cuts") (width 0.05))
 (gr_line (start 201.6788 109.3724) (end 201.6788 58.8724) (layer "Edge.Cuts") (width 0.05))
 (gr_arc (start 141.6788 75.8724) (mid 142.385907 76.165293) (end 142.6788 76.8724) (layer "Edge.Cuts") (width 0.05))
 (gr_line (start 137.6788 92.8724) (end 141.6788 92.8724) (layer "Edge.Cuts") (width 0.05))
 (gr_arc (start 139.6788 112.3724) (mid 137.55748 111.49372) (end 136.6788 109.3724) (layer "Edge.Cuts") (width 0.05))
 (gr_line (start 180.6788 108.3724) (end 180.6788 93.3724) (layer "Edge.Cuts") (width 0.05))
 (gr_line (start 140.6788 55.8724) (end 198.6788 55.8724) (layer "Edge.Cuts") (width 0.05))
 (gr_arc (start 136.6788 58.8724) (mid 137.55748 56.75108) (end 139.6788 55.8724) (layer "Edge.Cuts") (width 0.05))
 (gr_arc (start 182.6788 108.3724) (mid 181.6788 109.3724) (end 180.6788 108.3724) (layer "Edge.Cuts") (width 0.05))
 (gr_arc (start 198.6788 55.8724) (mid 200.80012 56.75108) (end 201.6788 58.8724) (layer "Edge.Cuts") (width 0.05))
 (gr_line (start 139.6788 112.3724) (end 140.6788 112.3724) (layer "Edge.Cuts") (width 0.05))
 (gr_line (start 139.6788 55.8724) (end 140.6788 55.8724) (layer "Edge.Cuts") (width 0.05))
 (gr_arc (start 136.6788 93.8724) (mid 136.971693 93.165293) (end 137.6788 92.8724) (layer "Edge.Cuts") (width 0.05))
 (gr_arc (start 180.6788 93.3724) (mid 181.6788 92.3724) (end 182.6788 93.3724) (layer "Edge.Cuts") (width 0.05))
 (segment (start 153.664 100.8216) (end 153.664 101.2656) (width 0.5) (layer "F.Cu") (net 3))
 (segment (start 164.7952 103.5456) (end 164.7596 103.5812) (width 0.5) (layer "F.Cu") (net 14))
 (segment (start 164.7952 101.5473) (end 164.7952 103.5456) (width 0.5) (layer "F.Cu") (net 14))
 (segment (start 163.5741 99.7223) (end 164.7952 99.7223) (width 0.5) (layer "F.Cu") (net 13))
 (segment (start 162.6362 100.6602) (end 163.5741 99.7223) (width 0.5) (layer "F.Cu") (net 13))
 (segment (start 166.9288 99.6848) (end 164.8327 99.6848) (width 0.5) (layer "F.Cu") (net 13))
 (segment (start 161.947598 100.6602) (end 162.6362 100.6602) (width 0.5) (layer "F.Cu") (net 13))
 (segment (start 166.8913 99.7223) (end 166.9288 99.6848) (width 0.5) (layer "F.Cu") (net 13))
 (segment (start 164.8327 99.6848) (end 164.7952 99.7223) (width 0.5) (layer "F.Cu") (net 13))
 (segment (start 173.9373 96.0628) (end 173.99 96.0101) (width 0.5) (layer "F.Cu") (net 7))
 (segment (start 141.4272 96.266) (end 149.6396 96.266) (width 3) (layer "F.Cu") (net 2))
 (segment (start 149.6396 96.266) (end 151.384 94.5216) (width 3) (layer "F.Cu") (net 2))
 (segment (start 153.170701 59.6126) (end 153.859 60.300899) (width 0.25) (layer "F.Cu") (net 19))
 (segment (start 148.969 59.6126) (end 153.170701 59.6126) (width 0.25) (layer "F.Cu") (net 19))
 (segment (start 153.859 60.300899) (end 153.859 61.1998) (width 0.25) (layer "F.Cu") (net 19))
 (segment (start 153.859 61.1998) (end 155.7528 63.0936) (width 0.25) (layer "F.Cu") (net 19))
 (segment (start 155.7528 63.0936) (end 159.4612 63.0936) (width 0.25) (layer "F.Cu") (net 19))
 (segment (start 159.4612 63.0936) (end 161.2392 64.8716) (width 0.25) (layer "F.Cu") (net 19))
 (segment (start 147.604 58.2476) (end 148.969 59.6126) (width 0.25) (layer "F.Cu") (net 19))
 (segment (start 161.2392 64.8716) (end 168.0028 64.8716) (width 0.25) (layer "F.Cu") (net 19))
 (segment (start 168.0028 64.8716) (end 170.7548 67.6236) (width 0.25) (layer "F.Cu") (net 19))
 (segment (start 156.589 61.274301) (end 156.589 60.4754) (width 0.25) (layer "F.Cu") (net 20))
 (segment (start 172.5764 67.6236) (end 168.8084 63.8556) (width 0.25) (layer "F.Cu") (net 20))
 (segment (start 154.852299 59.5376) (end 153.8732 58.558501) (width 0.25) (layer "F.Cu") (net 20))
 (segment (start 156.589 60.4754) (end 155.6512 59.5376) (width 0.25) (layer "F.Cu") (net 20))
 (segment (start 157.646299 62.3316) (end 156.589 61.274301) (width 0.25) (layer "F.Cu") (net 20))
 (segment (start 160.8836 63.8556) (end 159.3596 62.3316) (width 0.25) (layer "F.Cu") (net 20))
 (segment (start 155.6512 59.5376) (end 154.852299 59.5376) (width 0.25) (layer "F.Cu") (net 20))
 (segment (start 153.8732 58.558501) (end 153.8732 57.7088) (width 0.25) (layer "F.Cu") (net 20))
 (segment (start 150.7236 57.668) (end 150.144 58.2476) (width 0.25) (layer "F.Cu") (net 20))
 (segment (start 159.3596 62.3316) (end 157.646299 62.3316) (width 0.25) (layer "F.Cu") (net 20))
 (segment (start 153.162 56.9976) (end 150.7236 56.9976) (width 0.25) (layer "F.Cu") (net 20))
 (segment (start 153.8732 57.7088) (end 153.162 56.9976) (width 0.25) (layer "F.Cu") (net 20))
 (segment (start 168.8084 63.8556) (end 160.8836 63.8556) (width 0.25) (layer "F.Cu") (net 20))
 (segment (start 172.7548 67.6236) (end 172.5764 67.6236) (width 0.25) (layer "F.Cu") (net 20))
 (segment (start 150.7236 56.9976) (end 150.7236 57.668) (width 0.25) (layer "F.Cu") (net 20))
 (segment (start 181.989 67.5962) (end 181.989 59.6126) (width 0.25) (layer "F.Cu") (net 11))
 (segment (start 182.118 67.7252) (end 181.989 67.5962) (width 0.25) (layer "F.Cu") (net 11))
 (segment (start 181.989 59.6126) (end 180.624 58.2476) (width 0.25) (layer "F.Cu") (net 11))
 (segment (start 184.118 67.7252) (end 184.339 67.5042) (width 0.25) (layer "F.Cu") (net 12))
 (segment (start 184.339 67.5042) (end 184.339 59.620301) (width 0.25) (layer "F.Cu") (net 12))
 (segment (start 181.9656 58.710901) (end 181.9656 57.927499) (width 0.25) (layer "F.Cu") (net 12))
 (segment (start 181.9656 57.927499) (end 181.110701 57.0726) (width 0.25) (layer "F.Cu") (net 12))
 (segment (start 181.110701 57.0726) (end 179.259 57.0726) (width 0.25) (layer "F.Cu") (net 12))
 (segment (start 184.141299 59.4226) (end 182.677299 59.4226) (width 0.25) (layer "F.Cu") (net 12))
 (segment (start 182.677299 59.4226) (end 181.9656 58.710901) (width 0.25) (layer "F.Cu") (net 12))
 (segment (start 179.259 57.0726) (end 178.084 58.2476) (width 0.25) (layer "F.Cu") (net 12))
 (segment (start 184.339 59.620301) (end 184.141299 59.4226) (width 0.25) (layer "F.Cu") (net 12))
 (segment (start 159.0736 73.0711) (end 159.0736 67.564) (width 0.25) (layer "F.Cu") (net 17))
 (segment (start 159.7641 73.7616) (end 159.0736 73.0711) (width 0.25) (layer "F.Cu") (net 17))
 (segment (start 161.0736 66.3316) (end 158.4452 63.7032) (width 0.5) (layer "F.Cu") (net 18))
 (segment (start 158.4452 63.7032) (end 153.7208 63.7032) (width 0.5) (layer "F.Cu") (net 18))
 (segment (start 152.684 62.6664) (end 152.684 60.7876) (width 0.5) (layer "F.Cu") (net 18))
 (segment (start 153.7208 63.7032) (end 152.684 62.6664) (width 0.5) (layer "F.Cu") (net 18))
 (segment (start 161.0736 67.564) (end 161.0736 66.3316) (width 0.5) (layer "F.Cu") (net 18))
 (segment (start 155.224 72.8772) (end 156.1084 73.7616) (width 0.25) (layer "B.Cu") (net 23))
 (segment (start 155.224 60.7876) (end 155.224 72.8772) (width 0.25) (layer "B.Cu") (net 23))
 (segment (start 156.1084 73.7616) (end 157.9372 73.7616) (width 0.25) (layer "B.Cu") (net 23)))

